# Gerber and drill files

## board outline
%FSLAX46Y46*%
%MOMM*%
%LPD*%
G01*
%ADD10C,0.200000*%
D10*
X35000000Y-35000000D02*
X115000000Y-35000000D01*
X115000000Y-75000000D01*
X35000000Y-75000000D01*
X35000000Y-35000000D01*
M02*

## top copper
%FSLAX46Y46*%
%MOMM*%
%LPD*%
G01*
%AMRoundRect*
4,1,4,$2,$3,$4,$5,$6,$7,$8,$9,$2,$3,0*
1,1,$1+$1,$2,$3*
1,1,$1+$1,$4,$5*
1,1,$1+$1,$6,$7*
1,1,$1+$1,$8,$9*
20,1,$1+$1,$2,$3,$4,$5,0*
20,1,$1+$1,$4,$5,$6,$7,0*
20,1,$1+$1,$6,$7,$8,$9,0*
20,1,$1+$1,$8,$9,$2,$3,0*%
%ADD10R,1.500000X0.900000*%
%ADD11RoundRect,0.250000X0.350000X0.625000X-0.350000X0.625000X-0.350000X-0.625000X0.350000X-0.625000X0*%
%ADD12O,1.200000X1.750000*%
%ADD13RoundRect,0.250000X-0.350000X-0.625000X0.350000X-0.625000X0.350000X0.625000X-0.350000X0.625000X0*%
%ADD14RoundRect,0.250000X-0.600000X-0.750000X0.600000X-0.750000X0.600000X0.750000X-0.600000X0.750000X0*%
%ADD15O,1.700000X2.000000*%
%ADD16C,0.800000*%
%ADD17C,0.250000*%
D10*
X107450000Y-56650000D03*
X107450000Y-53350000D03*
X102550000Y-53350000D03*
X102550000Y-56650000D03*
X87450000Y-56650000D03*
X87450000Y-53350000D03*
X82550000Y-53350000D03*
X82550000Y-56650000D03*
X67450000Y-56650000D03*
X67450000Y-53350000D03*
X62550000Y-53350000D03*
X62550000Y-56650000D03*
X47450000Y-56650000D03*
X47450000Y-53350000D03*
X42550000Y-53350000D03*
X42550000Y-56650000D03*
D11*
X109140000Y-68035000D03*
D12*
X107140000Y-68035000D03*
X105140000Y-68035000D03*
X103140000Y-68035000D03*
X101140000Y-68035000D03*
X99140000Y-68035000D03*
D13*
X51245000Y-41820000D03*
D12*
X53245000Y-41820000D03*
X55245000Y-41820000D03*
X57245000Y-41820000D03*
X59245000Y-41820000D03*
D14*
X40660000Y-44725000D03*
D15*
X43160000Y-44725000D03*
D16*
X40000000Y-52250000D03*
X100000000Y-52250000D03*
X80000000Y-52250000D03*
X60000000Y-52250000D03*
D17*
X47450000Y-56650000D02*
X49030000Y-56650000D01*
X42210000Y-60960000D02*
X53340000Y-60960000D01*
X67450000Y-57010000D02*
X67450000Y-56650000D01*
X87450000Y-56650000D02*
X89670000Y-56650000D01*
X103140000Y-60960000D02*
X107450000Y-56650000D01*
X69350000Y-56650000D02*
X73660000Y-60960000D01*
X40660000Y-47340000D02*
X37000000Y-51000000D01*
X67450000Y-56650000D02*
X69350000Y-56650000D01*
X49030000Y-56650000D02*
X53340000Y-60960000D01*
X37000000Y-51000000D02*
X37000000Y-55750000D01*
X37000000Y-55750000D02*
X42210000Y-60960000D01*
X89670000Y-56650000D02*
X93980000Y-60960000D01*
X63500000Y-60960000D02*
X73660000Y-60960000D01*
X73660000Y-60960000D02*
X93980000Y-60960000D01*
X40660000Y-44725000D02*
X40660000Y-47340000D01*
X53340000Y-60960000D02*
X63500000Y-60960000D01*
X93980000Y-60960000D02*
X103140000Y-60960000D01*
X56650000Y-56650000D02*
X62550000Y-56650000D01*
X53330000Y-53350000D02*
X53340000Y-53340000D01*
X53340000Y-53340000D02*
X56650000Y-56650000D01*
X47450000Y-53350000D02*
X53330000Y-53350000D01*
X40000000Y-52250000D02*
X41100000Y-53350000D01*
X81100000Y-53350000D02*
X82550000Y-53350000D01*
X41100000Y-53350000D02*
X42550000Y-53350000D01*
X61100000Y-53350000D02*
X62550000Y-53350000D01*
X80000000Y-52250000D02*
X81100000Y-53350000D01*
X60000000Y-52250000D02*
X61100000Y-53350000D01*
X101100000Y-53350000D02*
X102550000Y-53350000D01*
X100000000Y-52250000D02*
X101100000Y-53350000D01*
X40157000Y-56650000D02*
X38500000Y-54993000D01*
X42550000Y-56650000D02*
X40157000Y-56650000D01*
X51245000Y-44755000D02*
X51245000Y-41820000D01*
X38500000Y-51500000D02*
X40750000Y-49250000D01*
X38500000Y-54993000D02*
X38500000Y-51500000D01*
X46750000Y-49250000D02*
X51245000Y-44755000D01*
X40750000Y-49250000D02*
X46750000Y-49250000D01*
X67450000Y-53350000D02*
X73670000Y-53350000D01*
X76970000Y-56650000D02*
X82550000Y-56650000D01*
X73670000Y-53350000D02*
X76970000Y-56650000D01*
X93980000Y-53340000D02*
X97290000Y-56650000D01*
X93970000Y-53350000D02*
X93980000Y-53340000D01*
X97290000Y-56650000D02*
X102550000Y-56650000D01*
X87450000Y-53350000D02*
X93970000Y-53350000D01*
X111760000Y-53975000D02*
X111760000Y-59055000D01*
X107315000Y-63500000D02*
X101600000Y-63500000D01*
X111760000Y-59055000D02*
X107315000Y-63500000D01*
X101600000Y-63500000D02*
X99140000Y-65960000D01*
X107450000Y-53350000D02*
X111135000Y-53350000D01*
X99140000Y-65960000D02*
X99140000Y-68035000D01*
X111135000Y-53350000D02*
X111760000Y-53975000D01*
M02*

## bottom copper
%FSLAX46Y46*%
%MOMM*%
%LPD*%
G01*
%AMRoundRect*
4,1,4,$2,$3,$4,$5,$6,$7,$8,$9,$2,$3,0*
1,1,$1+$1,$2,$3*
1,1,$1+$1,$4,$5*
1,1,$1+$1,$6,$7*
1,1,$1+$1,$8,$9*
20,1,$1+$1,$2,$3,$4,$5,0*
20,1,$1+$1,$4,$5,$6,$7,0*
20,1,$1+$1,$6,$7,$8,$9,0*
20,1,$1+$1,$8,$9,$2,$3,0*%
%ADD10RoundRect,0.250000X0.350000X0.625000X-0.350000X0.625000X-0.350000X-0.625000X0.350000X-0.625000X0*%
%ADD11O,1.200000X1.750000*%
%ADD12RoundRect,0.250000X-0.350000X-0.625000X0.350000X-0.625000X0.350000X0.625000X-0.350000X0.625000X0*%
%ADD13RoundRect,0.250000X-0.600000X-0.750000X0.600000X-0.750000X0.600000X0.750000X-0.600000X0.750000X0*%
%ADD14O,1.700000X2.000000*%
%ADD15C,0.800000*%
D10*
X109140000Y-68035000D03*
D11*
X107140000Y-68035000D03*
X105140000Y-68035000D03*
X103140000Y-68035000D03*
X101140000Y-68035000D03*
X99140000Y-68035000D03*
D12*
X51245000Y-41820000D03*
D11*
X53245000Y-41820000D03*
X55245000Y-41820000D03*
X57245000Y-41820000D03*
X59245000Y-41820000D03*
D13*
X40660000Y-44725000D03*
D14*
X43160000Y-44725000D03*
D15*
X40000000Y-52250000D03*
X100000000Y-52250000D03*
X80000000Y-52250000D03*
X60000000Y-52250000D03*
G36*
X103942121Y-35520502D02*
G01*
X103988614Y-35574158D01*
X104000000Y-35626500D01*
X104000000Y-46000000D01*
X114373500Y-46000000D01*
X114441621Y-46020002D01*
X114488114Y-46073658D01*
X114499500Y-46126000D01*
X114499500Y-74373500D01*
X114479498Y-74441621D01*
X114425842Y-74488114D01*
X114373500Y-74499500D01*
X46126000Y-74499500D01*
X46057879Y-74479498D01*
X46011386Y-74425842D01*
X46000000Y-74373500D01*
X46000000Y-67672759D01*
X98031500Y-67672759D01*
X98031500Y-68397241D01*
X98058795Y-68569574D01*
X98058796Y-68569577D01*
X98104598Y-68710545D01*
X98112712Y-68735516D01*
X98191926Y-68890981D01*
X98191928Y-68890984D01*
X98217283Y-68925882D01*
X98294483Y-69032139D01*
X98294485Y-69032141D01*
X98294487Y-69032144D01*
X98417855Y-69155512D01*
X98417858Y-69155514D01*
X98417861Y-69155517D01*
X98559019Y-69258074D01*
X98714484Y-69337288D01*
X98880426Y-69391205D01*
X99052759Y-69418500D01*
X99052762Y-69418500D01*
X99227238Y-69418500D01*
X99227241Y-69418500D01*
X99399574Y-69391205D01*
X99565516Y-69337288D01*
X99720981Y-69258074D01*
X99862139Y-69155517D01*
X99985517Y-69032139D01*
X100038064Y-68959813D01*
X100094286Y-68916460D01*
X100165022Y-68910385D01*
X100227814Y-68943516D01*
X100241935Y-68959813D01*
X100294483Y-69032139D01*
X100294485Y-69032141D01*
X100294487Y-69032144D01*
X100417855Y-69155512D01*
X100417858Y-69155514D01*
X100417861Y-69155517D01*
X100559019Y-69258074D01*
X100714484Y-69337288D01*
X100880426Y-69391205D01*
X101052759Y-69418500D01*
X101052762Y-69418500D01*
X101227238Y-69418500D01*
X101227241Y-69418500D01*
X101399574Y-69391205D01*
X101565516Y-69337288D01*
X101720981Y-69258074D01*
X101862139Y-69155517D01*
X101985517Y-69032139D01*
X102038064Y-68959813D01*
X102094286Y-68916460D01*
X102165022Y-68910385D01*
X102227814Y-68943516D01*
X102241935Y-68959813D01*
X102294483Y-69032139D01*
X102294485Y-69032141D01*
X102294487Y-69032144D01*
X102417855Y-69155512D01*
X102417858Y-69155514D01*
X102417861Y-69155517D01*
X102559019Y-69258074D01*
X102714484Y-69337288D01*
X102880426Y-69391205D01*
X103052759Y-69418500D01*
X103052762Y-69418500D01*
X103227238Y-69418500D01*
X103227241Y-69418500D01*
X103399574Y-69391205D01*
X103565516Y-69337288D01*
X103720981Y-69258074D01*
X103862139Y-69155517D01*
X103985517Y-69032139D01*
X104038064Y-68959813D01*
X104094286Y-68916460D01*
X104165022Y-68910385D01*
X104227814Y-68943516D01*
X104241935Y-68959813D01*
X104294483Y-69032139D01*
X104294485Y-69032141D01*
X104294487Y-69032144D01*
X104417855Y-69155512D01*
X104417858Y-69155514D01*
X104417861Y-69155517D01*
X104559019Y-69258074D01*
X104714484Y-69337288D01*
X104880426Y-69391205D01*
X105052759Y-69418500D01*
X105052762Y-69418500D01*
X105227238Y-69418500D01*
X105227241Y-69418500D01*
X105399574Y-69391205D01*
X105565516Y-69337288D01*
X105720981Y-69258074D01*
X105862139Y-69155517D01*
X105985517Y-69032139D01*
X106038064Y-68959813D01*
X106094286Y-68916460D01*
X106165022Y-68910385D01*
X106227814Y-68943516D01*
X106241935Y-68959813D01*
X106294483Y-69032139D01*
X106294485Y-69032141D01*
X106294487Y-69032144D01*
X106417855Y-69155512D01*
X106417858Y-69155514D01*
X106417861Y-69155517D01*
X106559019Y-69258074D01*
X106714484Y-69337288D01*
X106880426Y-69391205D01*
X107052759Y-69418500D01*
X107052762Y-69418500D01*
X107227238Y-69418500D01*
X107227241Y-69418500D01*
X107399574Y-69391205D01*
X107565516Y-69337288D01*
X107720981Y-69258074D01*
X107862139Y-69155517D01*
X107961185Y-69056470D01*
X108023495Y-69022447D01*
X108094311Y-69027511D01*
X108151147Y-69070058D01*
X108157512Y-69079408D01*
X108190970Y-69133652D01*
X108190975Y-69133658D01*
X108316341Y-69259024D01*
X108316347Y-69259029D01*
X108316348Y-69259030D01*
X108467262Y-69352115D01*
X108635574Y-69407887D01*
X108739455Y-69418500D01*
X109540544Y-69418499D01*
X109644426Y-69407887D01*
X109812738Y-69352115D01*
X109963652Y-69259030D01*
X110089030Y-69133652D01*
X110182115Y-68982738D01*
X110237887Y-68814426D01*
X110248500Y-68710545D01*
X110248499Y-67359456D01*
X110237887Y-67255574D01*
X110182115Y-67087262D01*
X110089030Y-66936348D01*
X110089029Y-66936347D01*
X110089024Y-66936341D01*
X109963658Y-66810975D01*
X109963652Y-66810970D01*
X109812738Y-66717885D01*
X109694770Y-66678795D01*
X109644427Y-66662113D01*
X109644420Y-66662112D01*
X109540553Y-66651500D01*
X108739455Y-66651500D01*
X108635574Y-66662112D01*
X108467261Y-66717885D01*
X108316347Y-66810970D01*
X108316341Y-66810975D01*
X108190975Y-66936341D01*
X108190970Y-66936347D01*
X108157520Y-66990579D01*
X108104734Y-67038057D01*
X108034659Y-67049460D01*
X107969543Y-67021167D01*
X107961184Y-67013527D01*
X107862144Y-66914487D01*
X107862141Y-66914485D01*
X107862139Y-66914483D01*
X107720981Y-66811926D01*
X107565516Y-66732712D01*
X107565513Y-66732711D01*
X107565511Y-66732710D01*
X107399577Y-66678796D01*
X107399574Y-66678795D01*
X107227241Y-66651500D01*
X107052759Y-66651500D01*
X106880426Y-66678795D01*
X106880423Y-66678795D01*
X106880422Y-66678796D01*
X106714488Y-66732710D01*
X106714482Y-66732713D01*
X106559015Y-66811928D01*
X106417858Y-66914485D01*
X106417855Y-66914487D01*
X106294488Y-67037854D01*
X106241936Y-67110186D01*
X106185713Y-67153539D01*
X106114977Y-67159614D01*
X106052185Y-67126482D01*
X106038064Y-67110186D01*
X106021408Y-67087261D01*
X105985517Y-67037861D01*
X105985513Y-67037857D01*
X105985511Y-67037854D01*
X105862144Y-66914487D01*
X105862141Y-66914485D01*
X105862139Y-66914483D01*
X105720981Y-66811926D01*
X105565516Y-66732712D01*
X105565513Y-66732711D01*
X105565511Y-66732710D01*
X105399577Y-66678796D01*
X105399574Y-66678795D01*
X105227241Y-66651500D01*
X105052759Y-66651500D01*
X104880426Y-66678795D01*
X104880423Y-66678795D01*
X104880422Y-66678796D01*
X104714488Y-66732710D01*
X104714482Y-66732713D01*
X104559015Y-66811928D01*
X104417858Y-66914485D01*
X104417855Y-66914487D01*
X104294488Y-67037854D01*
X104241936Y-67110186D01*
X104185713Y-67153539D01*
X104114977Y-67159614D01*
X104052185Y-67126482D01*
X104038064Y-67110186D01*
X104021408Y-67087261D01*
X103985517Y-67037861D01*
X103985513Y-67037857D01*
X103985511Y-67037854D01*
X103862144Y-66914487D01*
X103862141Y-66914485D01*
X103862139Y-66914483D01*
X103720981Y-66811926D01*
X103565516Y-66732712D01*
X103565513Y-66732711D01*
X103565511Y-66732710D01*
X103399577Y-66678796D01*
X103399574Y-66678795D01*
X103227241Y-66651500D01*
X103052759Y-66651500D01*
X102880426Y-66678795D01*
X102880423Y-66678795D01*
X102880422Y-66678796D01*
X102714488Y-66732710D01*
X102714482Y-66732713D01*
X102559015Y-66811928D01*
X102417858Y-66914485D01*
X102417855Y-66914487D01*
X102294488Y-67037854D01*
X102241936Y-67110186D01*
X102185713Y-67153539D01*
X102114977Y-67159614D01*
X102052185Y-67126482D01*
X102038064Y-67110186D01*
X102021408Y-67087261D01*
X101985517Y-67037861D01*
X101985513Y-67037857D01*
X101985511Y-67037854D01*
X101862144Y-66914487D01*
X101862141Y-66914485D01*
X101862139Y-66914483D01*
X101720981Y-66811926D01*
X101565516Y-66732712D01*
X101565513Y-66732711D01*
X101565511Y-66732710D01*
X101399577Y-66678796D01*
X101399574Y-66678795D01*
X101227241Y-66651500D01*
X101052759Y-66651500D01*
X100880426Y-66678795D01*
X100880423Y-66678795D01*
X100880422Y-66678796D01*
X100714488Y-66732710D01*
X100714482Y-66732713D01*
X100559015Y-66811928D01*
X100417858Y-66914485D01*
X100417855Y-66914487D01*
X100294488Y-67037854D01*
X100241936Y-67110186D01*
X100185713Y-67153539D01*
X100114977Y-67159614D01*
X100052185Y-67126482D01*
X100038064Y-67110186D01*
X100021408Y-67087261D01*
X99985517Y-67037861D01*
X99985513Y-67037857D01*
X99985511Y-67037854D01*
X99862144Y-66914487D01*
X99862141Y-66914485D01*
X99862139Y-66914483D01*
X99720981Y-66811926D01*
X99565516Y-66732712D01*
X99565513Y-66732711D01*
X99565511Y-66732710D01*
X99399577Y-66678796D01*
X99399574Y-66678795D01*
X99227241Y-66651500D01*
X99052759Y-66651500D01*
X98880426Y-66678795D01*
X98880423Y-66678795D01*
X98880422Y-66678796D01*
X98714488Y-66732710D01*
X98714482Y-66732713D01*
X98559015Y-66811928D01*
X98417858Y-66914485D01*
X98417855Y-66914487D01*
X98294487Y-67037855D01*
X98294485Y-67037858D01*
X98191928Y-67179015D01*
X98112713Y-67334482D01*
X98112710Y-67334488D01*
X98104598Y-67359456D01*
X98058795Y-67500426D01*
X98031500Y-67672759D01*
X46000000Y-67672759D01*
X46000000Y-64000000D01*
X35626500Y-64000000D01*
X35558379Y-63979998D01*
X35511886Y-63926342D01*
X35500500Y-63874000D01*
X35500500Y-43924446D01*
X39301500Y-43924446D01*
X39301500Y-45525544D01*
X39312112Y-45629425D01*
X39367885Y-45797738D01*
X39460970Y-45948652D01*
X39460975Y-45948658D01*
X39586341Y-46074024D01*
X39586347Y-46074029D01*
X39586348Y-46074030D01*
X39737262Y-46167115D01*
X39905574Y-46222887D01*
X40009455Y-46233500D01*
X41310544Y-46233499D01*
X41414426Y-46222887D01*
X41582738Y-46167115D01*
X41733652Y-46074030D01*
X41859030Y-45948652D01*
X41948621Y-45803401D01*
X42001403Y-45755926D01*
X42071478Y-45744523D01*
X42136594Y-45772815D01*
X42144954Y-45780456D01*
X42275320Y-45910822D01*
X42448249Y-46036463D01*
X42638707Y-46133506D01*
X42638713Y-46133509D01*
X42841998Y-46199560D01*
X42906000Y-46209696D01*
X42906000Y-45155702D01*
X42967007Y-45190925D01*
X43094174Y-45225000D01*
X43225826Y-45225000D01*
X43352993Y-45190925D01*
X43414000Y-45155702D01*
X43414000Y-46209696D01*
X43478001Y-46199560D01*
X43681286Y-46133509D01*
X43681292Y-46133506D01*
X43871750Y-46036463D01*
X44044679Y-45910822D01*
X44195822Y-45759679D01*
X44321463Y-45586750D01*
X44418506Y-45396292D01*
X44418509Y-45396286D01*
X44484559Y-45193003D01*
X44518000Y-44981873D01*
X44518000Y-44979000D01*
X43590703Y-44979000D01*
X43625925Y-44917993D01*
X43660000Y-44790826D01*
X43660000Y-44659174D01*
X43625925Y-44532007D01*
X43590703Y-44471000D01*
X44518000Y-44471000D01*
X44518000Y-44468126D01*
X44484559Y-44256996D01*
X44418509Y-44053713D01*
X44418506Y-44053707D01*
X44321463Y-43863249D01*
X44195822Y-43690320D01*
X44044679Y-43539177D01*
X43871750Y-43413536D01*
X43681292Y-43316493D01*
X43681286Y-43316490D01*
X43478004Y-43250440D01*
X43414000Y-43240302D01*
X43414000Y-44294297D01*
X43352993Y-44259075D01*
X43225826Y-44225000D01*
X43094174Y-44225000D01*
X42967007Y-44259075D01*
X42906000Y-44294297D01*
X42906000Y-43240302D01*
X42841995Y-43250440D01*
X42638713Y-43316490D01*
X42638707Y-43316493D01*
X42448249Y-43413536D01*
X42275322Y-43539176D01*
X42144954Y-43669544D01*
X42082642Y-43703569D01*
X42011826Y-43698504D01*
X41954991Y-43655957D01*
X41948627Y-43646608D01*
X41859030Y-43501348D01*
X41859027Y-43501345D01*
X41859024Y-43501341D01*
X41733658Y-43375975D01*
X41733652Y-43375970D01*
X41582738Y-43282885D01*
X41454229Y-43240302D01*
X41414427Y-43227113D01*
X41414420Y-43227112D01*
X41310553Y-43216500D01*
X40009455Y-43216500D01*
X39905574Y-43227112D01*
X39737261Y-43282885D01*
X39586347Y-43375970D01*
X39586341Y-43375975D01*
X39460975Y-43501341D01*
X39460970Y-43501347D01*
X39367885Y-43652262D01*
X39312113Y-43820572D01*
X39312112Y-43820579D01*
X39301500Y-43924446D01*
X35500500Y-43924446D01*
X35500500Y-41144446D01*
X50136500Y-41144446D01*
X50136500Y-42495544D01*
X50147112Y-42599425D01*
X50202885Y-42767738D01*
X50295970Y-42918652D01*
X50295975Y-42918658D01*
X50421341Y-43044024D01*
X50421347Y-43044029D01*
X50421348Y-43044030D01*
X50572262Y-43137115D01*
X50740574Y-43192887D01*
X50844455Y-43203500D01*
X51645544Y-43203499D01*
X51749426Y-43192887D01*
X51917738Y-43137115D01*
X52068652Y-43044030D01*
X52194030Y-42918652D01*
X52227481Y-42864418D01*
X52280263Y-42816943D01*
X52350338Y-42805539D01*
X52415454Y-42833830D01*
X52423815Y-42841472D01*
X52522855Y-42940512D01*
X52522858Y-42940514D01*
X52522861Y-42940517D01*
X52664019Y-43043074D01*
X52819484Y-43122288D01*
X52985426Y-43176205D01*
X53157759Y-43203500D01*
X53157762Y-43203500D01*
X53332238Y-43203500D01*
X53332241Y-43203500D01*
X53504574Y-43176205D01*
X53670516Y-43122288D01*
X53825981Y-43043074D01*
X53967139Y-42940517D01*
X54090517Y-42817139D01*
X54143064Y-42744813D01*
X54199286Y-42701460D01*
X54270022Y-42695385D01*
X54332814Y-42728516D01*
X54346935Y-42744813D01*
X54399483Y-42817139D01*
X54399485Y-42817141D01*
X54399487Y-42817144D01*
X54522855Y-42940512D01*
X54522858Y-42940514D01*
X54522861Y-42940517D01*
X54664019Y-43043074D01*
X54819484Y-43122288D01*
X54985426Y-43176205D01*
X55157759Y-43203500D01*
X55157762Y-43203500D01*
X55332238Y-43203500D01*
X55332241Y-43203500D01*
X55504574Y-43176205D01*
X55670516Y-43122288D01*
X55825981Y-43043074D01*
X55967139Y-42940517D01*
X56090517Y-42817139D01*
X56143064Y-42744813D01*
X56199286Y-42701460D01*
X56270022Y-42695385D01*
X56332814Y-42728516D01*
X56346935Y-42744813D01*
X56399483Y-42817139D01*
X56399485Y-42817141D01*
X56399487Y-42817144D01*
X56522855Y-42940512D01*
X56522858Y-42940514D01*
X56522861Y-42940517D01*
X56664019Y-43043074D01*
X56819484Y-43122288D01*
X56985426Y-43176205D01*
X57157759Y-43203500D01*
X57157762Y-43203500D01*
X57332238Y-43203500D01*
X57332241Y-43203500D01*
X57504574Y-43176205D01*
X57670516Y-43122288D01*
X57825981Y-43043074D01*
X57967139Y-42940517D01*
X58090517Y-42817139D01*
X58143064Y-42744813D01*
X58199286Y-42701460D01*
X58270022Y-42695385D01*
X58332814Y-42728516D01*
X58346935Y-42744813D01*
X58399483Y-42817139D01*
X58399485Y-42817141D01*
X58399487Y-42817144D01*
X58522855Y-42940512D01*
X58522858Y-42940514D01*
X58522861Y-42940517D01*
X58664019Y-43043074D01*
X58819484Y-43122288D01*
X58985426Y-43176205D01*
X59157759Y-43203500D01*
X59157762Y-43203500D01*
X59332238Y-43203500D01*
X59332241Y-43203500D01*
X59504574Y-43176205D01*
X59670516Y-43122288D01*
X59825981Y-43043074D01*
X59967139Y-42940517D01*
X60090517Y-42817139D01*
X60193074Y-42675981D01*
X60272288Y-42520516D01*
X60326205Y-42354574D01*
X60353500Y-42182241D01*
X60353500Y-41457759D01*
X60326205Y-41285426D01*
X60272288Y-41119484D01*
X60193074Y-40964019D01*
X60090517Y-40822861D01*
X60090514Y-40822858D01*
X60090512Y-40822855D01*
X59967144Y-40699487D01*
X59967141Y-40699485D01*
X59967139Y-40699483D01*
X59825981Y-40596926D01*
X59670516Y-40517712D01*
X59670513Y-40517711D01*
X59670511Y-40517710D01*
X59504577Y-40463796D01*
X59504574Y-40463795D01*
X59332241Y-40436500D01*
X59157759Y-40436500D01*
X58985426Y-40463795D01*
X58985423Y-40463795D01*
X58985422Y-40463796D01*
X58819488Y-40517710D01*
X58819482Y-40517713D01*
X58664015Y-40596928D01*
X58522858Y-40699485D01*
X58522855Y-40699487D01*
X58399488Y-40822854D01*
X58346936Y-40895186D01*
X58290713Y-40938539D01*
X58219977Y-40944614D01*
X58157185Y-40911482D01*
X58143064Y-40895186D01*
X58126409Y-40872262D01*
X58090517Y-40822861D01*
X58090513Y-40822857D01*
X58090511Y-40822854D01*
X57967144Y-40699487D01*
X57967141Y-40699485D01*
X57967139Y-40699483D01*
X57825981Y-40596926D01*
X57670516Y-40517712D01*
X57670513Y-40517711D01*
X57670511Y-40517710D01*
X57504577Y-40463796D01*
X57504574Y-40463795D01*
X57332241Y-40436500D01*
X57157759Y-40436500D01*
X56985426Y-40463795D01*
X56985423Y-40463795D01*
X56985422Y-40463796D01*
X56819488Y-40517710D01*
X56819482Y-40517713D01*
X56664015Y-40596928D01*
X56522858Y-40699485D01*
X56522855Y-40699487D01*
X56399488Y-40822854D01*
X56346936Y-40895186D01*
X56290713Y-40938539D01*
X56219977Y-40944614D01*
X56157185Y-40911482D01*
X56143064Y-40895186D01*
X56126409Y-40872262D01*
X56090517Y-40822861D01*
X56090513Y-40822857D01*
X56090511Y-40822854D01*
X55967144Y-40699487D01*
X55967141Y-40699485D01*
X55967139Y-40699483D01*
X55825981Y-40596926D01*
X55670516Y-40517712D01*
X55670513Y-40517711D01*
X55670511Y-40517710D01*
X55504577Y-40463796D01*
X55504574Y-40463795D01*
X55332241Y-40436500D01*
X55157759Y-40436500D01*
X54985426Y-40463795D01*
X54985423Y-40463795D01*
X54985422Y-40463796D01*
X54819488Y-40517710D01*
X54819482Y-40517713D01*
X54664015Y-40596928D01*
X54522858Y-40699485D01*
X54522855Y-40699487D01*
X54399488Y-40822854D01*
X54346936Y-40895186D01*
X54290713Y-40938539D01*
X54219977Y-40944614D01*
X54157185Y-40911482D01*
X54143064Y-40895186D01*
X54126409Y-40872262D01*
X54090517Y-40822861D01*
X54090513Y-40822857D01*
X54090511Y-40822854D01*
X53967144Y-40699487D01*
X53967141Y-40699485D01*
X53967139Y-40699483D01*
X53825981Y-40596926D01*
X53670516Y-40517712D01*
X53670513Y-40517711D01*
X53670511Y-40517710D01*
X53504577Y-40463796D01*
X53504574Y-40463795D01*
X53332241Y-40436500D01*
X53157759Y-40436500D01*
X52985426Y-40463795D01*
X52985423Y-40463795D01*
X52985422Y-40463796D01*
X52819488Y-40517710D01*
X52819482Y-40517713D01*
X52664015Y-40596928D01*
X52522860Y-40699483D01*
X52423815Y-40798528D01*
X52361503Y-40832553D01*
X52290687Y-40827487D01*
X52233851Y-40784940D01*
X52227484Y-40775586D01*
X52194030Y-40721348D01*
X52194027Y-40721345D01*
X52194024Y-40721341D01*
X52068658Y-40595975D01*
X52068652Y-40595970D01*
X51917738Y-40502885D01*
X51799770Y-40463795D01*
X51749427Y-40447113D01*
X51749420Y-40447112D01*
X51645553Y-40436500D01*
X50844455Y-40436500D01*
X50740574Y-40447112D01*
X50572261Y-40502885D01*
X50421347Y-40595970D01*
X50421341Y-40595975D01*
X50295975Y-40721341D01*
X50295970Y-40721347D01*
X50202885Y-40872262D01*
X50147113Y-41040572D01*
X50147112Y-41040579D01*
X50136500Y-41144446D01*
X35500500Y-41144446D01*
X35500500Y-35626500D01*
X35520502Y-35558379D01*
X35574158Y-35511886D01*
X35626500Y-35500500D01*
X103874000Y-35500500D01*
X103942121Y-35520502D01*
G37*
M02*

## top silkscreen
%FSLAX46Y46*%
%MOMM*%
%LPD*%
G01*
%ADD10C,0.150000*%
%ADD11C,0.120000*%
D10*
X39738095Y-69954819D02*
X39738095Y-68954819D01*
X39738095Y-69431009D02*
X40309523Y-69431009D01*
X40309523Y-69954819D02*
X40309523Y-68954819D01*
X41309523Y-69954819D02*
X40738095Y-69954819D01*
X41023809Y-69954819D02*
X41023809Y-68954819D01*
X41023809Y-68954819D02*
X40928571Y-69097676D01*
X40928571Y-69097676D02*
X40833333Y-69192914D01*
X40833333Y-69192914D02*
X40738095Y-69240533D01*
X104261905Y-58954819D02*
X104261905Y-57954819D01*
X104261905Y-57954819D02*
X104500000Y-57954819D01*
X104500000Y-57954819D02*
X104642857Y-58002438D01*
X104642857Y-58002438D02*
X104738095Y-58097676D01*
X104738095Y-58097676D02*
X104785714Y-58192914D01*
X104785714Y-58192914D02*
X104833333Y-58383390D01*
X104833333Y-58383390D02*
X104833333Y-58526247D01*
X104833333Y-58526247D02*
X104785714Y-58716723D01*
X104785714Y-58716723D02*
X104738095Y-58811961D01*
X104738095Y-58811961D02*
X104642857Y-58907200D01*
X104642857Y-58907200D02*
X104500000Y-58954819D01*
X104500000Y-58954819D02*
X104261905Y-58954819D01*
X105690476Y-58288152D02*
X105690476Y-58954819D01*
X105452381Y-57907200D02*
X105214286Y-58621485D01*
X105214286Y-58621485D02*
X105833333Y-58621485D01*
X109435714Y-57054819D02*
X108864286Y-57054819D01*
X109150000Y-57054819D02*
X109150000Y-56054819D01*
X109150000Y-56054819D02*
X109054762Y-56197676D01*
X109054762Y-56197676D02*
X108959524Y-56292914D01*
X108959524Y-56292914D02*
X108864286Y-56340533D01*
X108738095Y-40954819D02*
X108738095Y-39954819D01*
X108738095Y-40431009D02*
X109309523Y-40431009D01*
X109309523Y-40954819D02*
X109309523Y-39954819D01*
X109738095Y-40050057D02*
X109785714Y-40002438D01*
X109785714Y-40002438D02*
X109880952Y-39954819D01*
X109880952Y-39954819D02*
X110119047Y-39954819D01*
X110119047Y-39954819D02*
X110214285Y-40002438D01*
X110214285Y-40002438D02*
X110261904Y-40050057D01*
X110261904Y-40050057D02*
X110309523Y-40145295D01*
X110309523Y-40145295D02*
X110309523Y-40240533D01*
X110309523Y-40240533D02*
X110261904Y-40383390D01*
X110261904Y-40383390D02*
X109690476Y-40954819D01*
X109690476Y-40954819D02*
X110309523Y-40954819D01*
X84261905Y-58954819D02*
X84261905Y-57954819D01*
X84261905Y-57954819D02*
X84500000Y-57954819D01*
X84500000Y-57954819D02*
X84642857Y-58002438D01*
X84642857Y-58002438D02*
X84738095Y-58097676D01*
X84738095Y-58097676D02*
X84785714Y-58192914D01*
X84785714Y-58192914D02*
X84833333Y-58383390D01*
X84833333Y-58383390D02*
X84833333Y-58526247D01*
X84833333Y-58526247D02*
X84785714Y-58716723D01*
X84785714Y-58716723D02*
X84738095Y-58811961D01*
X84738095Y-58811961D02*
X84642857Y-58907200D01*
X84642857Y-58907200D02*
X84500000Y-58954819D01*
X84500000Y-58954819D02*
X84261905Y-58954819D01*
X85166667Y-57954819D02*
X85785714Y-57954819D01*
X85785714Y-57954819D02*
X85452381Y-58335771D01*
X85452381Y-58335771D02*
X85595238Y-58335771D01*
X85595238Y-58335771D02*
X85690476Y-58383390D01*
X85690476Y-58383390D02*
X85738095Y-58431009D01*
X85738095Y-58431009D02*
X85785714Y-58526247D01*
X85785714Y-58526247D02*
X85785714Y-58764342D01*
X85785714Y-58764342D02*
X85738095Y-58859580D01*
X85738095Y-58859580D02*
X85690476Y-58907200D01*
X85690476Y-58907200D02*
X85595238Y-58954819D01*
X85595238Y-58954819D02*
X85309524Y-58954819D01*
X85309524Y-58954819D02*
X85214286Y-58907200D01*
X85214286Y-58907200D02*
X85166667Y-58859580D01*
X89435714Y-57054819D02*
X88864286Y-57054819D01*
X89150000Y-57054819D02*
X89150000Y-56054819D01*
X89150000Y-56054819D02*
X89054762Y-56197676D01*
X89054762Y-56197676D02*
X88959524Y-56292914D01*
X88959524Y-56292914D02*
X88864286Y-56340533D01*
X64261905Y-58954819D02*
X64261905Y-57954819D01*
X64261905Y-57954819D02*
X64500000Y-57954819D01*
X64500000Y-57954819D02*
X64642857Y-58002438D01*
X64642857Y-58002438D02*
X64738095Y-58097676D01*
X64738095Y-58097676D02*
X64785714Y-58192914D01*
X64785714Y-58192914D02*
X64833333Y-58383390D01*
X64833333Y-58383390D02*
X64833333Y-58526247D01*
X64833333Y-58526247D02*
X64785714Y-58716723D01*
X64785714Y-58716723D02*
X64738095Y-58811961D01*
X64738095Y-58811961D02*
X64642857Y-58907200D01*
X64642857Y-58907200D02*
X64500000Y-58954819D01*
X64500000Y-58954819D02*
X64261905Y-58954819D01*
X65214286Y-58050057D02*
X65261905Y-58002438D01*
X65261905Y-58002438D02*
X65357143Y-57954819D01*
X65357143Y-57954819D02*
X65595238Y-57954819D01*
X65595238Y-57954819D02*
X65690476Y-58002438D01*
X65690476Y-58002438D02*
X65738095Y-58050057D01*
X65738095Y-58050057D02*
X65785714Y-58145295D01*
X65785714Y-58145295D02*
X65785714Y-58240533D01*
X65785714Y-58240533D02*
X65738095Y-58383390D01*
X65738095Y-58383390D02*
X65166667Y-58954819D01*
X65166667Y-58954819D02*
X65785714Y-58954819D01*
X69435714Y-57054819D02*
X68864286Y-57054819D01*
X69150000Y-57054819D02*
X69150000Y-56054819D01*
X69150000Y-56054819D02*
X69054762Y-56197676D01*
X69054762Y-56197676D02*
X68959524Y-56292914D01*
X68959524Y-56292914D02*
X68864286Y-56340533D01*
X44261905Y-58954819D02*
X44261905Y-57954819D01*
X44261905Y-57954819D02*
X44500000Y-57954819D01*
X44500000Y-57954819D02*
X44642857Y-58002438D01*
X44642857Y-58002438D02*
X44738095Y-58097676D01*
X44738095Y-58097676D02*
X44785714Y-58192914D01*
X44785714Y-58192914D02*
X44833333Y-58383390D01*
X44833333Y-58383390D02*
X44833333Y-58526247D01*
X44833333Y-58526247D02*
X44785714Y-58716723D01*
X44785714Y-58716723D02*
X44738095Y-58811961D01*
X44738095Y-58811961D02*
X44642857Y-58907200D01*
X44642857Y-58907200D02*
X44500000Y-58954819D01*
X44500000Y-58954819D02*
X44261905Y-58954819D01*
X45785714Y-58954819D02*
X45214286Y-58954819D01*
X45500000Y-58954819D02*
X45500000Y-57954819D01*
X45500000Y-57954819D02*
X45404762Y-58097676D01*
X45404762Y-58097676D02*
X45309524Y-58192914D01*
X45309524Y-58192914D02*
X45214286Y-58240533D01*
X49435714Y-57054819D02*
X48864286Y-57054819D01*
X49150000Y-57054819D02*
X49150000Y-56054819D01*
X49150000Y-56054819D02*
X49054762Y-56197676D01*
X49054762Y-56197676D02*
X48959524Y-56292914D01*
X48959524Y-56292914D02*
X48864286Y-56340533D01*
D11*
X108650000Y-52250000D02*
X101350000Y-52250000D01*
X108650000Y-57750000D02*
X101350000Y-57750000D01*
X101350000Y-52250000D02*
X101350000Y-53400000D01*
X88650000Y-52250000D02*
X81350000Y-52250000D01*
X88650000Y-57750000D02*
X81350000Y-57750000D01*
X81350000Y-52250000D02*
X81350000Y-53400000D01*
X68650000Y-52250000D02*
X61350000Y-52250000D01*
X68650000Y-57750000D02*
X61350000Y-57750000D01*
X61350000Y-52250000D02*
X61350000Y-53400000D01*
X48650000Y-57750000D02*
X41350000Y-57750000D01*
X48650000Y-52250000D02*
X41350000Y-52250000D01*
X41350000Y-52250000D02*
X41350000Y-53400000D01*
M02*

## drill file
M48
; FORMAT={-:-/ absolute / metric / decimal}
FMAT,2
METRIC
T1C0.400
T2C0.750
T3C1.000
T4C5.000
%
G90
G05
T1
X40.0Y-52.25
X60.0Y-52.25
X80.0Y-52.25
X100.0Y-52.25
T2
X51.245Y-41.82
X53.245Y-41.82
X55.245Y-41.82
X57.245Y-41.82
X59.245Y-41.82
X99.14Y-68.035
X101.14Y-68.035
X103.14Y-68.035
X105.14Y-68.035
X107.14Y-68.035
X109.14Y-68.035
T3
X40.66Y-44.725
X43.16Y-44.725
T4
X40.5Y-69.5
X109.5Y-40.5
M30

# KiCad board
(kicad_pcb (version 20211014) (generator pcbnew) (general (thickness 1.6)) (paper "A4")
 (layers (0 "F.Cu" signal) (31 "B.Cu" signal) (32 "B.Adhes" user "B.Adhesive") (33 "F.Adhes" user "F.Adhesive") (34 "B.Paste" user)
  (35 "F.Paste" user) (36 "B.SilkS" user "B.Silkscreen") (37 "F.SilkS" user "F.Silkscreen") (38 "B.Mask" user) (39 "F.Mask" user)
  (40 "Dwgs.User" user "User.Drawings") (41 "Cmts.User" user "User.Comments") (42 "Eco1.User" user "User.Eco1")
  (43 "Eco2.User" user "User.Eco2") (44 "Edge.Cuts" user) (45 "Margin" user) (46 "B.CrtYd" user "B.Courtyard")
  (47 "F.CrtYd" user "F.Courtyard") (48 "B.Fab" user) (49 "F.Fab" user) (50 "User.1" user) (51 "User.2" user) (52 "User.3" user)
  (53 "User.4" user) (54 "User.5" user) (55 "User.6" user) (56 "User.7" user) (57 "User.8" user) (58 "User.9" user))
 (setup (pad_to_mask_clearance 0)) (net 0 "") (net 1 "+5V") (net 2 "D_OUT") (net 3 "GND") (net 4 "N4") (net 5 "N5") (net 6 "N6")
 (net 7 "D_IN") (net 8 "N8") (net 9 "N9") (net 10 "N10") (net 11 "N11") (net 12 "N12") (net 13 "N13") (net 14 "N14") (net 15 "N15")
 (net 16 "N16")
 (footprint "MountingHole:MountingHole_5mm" (layer "F.Cu") (at 40.5 69.5)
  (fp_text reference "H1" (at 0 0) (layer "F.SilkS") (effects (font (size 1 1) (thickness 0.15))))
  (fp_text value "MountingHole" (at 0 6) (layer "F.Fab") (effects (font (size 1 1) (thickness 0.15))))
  (pad "" np_thru_hole circle (at 0 0) (size 5 5) (drill 5) (layers *.Cu *.Mask)))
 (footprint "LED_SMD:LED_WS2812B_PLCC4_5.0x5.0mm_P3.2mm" (layer "F.Cu") (at 105 55 180)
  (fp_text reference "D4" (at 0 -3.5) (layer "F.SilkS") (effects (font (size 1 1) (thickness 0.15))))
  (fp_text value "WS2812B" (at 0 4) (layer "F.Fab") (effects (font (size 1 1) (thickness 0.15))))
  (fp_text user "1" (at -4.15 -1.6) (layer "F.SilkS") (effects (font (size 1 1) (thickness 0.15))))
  (fp_line (start -3.65 2.75) (end 3.65 2.75) (layer "F.SilkS") (width 0.12))
  (fp_line (start -3.65 -2.75) (end 3.65 -2.75) (layer "F.SilkS") (width 0.12))
  (fp_line (start 3.65 2.75) (end 3.65 1.6) (layer "F.SilkS") (width 0.12))
  (pad "1" smd rect (at -2.45 -1.65 180) (size 1.5 0.9) (layers "F.Cu" "F.Paste" "F.Mask") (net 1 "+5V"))
  (pad "2" smd rect (at -2.45 1.65 180) (size 1.5 0.9) (layers "F.Cu" "F.Paste" "F.Mask") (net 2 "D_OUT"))
  (pad "3" smd rect (at 2.45 1.65 180) (size 1.5 0.9) (layers "F.Cu" "F.Paste" "F.Mask") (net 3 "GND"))
  (pad "4" smd rect (at 2.45 -1.65 180) (size 1.5 0.9) (layers "F.Cu" "F.Paste" "F.Mask") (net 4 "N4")))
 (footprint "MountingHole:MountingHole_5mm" (layer "F.Cu") (at 109.5 40.5)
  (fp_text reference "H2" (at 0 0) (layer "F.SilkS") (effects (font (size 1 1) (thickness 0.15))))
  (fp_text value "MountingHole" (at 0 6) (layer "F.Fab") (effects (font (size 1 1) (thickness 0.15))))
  (pad "" np_thru_hole circle (at 0 0) (size 5 5) (drill 5) (layers *.Cu *.Mask)))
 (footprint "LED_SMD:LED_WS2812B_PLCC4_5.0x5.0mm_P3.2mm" (layer "F.Cu") (at 85 55 180)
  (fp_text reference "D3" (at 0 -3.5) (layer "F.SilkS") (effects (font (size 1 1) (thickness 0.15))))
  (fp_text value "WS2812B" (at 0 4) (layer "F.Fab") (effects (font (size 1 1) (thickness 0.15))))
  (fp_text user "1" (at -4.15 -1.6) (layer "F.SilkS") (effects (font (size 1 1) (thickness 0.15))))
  (fp_line (start -3.65 2.75) (end 3.65 2.75) (layer "F.SilkS") (width 0.12))
  (fp_line (start -3.65 -2.75) (end 3.65 -2.75) (layer "F.SilkS") (width 0.12))
  (fp_line (start 3.65 2.75) (end 3.65 1.6) (layer "F.SilkS") (width 0.12))
  (pad "1" smd rect (at -2.45 -1.65 180) (size 1.5 0.9) (layers "F.Cu" "F.Paste" "F.Mask") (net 1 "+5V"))
  (pad "2" smd rect (at -2.45 1.65 180) (size 1.5 0.9) (layers "F.Cu" "F.Paste" "F.Mask") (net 4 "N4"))
  (pad "3" smd rect (at 2.45 1.65 180) (size 1.5 0.9) (layers "F.Cu" "F.Paste" "F.Mask") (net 3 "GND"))
  (pad "4" smd rect (at 2.45 -1.65 180) (size 1.5 0.9) (layers "F.Cu" "F.Paste" "F.Mask") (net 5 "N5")))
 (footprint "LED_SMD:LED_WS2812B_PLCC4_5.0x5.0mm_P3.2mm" (layer "F.Cu") (at 65 55 180)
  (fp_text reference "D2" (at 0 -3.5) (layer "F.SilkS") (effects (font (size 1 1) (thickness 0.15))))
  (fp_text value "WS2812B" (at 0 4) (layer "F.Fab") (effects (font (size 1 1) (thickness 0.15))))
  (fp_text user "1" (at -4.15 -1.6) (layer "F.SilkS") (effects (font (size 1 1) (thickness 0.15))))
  (fp_line (start -3.65 2.75) (end 3.65 2.75) (layer "F.SilkS") (width 0.12))
  (fp_line (start -3.65 -2.75) (end 3.65 -2.75) (layer "F.SilkS") (width 0.12))
  (fp_line (start 3.65 2.75) (end 3.65 1.6) (layer "F.SilkS") (width 0.12))
  (pad "1" smd rect (at -2.45 -1.65 180) (size 1.5 0.9) (layers "F.Cu" "F.Paste" "F.Mask") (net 1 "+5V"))
  (pad "2" smd rect (at -2.45 1.65 180) (size 1.5 0.9) (layers "F.Cu" "F.Paste" "F.Mask") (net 5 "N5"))
  (pad "3" smd rect (at 2.45 1.65 180) (size 1.5 0.9) (layers "F.Cu" "F.Paste" "F.Mask") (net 3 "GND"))
  (pad "4" smd rect (at 2.45 -1.65 180) (size 1.5 0.9) (layers "F.Cu" "F.Paste" "F.Mask") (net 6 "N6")))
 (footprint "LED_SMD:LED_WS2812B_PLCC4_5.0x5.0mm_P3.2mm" (layer "F.Cu") (at 45 55 180)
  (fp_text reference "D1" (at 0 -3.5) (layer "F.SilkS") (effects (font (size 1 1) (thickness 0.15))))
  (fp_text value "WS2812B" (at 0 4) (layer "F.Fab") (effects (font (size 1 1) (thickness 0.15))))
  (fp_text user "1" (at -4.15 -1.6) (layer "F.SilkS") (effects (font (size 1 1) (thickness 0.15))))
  (fp_line (start -3.65 -2.75) (end 3.65 -2.75) (layer "F.SilkS") (width 0.12))
  (fp_line (start -3.65 2.75) (end 3.65 2.75) (layer "F.SilkS") (width 0.12))
  (fp_line (start 3.65 2.75) (end 3.65 1.6) (layer "F.SilkS") (width 0.12))
  (pad "1" smd rect (at -2.45 -1.65 180) (size 1.5 0.9) (layers "F.Cu" "F.Paste" "F.Mask") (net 1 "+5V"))
  (pad "2" smd rect (at -2.45 1.65 180) (size 1.5 0.9) (layers "F.Cu" "F.Paste" "F.Mask") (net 6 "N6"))
  (pad "3" smd rect (at 2.45 1.65 180) (size 1.5 0.9) (layers "F.Cu" "F.Paste" "F.Mask") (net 3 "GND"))
  (pad "4" smd rect (at 2.45 -1.65 180) (size 1.5 0.9) (layers "F.Cu" "F.Paste" "F.Mask") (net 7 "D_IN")))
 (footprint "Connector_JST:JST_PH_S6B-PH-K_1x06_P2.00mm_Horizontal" (layer "B.Cu") (at 109.14 68.035 180)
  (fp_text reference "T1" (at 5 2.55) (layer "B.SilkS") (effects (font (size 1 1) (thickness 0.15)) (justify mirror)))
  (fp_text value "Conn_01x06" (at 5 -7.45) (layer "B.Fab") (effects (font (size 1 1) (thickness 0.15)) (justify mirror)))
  (pad "1" thru_hole roundrect (at 0 0 180) (size 1.2 1.75) (drill 0.75) (layers *.Cu *.Mask) (roundrect_rratio 0.2083333333) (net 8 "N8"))
  (pad "2" thru_hole oval (at 2 0 180) (size 1.2 1.75) (drill 0.75) (layers *.Cu *.Mask) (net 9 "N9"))
  (pad "3" thru_hole oval (at 4 0 180) (size 1.2 1.75) (drill 0.75) (layers *.Cu *.Mask) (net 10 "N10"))
  (pad "4" thru_hole oval (at 6 0 180) (size 1.2 1.75) (drill 0.75) (layers *.Cu *.Mask) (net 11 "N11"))
  (pad "5" thru_hole oval (at 8 0 180) (size 1.2 1.75) (drill 0.75) (layers *.Cu *.Mask) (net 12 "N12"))
  (pad "6" thru_hole oval (at 10 0 180) (size 1.2 1.75) (drill 0.75) (layers *.Cu *.Mask) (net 2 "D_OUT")))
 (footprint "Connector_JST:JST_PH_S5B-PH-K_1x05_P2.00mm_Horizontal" (layer "B.Cu") (at 51.245 41.82)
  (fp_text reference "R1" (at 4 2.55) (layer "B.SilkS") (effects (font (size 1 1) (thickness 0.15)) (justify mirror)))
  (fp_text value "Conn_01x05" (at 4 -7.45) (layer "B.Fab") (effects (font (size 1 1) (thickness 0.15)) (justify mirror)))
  (pad "1" thru_hole roundrect (at 0 0) (size 1.2 1.75) (drill 0.75) (layers *.Cu *.Mask) (roundrect_rratio 0.2083333333) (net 7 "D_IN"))
  (pad "2" thru_hole oval (at 2 0) (size 1.2 1.75) (drill 0.75) (layers *.Cu *.Mask) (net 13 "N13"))
  (pad "3" thru_hole oval (at 4 0) (size 1.2 1.75) (drill 0.75) (layers *.Cu *.Mask) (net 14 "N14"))
  (pad "4" thru_hole oval (at 6 0) (size 1.2 1.75) (drill 0.75) (layers *.Cu *.Mask) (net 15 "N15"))
  (pad "5" thru_hole oval (at 8 0) (size 1.2 1.75) (drill 0.75) (layers *.Cu *.Mask) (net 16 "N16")))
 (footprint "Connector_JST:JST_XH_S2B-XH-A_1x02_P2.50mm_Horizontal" (layer "B.Cu") (at 40.66 44.725)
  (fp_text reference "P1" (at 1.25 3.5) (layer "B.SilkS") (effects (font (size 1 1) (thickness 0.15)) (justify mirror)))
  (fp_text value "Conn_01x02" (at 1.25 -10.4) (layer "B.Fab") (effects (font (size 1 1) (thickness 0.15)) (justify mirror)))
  (pad "1" thru_hole roundrect (at 0 0) (size 1.7 2) (drill 1) (layers *.Cu *.Mask) (roundrect_rratio 0.1470588235) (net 1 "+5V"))
  (pad "2" thru_hole oval (at 2.5 0) (size 1.7 2) (drill 1) (layers *.Cu *.Mask) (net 3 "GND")))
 (gr_rect (start 35 35) (end 115 75) (layer "Edge.Cuts") (width 0.2) (fill none))
 (segment (start 47.45 56.65) (end 49.03 56.65) (width 0.25) (layer "F.Cu") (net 1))
 (segment (start 42.21 60.96) (end 53.34 60.96) (width 0.25) (layer "F.Cu") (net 1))
 (segment (start 67.45 57.01) (end 67.45 56.65) (width 0.25) (layer "F.Cu") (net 1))
 (segment (start 87.45 56.65) (end 89.67 56.65) (width 0.25) (layer "F.Cu") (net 1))
 (segment (start 103.14 60.96) (end 107.45 56.65) (width 0.25) (layer "F.Cu") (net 1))
 (segment (start 69.35 56.65) (end 73.66 60.96) (width 0.25) (layer "F.Cu") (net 1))
 (segment (start 40.66 47.34) (end 37 51) (width 0.25) (layer "F.Cu") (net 1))
 (segment (start 67.45 56.65) (end 69.35 56.65) (width 0.25) (layer "F.Cu") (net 1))
 (segment (start 49.03 56.65) (end 53.34 60.96) (width 0.25) (layer "F.Cu") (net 1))
 (segment (start 37 51) (end 37 55.75) (width 0.25) (layer "F.Cu") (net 1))
 (segment (start 37 55.75) (end 42.21 60.96) (width 0.25) (layer "F.Cu") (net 1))
 (segment (start 89.67 56.65) (end 93.98 60.96) (width 0.25) (layer "F.Cu") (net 1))
 (segment (start 63.5 60.96) (end 73.66 60.96) (width 0.25) (layer "F.Cu") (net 1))
 (segment (start 73.66 60.96) (end 93.98 60.96) (width 0.25) (layer "F.Cu") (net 1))
 (segment (start 40.66 44.725) (end 40.66 47.34) (width 0.25) (layer "F.Cu") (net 1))
 (segment (start 53.34 60.96) (end 63.5 60.96) (width 0.25) (layer "F.Cu") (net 1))
 (segment (start 93.98 60.96) (end 103.14 60.96) (width 0.25) (layer "F.Cu") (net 1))
 (segment (start 56.65 56.65) (end 62.55 56.65) (width 0.25) (layer "F.Cu") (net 6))
 (segment (start 53.33 53.35) (end 53.34 53.34) (width 0.25) (layer "F.Cu") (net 6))
 (segment (start 53.34 53.34) (end 56.65 56.65) (width 0.25) (layer "F.Cu") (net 6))
 (segment (start 47.45 53.35) (end 53.33 53.35) (width 0.25) (layer "F.Cu") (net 6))
 (segment (start 40 52.25) (end 41.1 53.35) (width 0.25) (layer "F.Cu") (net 3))
 (segment (start 81.1 53.35) (end 82.55 53.35) (width 0.25) (layer "F.Cu") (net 3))
 (segment (start 41.1 53.35) (end 42.55 53.35) (width 0.25) (layer "F.Cu") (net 3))
 (segment (start 61.1 53.35) (end 62.55 53.35) (width 0.25) (layer "F.Cu") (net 3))
 (segment (start 80 52.25) (end 81.1 53.35) (width 0.25) (layer "F.Cu") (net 3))
 (segment (start 60 52.25) (end 61.1 53.35) (width 0.25) (layer "F.Cu") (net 3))
 (segment (start 101.1 53.35) (end 102.55 53.35) (width 0.25) (layer "F.Cu") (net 3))
 (segment (start 100 52.25) (end 101.1 53.35) (width 0.25) (layer "F.Cu") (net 3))
 (via (at 40 52.25) (size 0.8) (drill 0.4) (layers "F.Cu" "B.Cu") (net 3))
 (via (at 100 52.25) (size 0.8) (drill 0.4) (layers "F.Cu" "B.Cu") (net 3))
 (via (at 80 52.25) (size 0.8) (drill 0.4) (layers "F.Cu" "B.Cu") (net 3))
 (via (at 60 52.25) (size 0.8) (drill 0.4) (layers "F.Cu" "B.Cu") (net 3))
 (segment (start 40.157 56.65) (end 38.5 54.993) (width 0.25) (layer "F.Cu") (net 7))
 (segment (start 42.55 56.65) (end 40.157 56.65) (width 0.25) (layer "F.Cu") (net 7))
 (segment (start 51.245 44.755) (end 51.245 41.82) (width 0.25) (layer "F.Cu") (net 7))
 (segment (start 38.5 51.5) (end 40.75 49.25) (width 0.25) (layer "F.Cu") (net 7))
 (segment (start 38.5 54.993) (end 38.5 51.5) (width 0.25) (layer "F.Cu") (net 7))
 (segment (start 46.75 49.25) (end 51.245 44.755) (width 0.25) (layer "F.Cu") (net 7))
 (segment (start 40.75 49.25) (end 46.75 49.25) (width 0.25) (layer "F.Cu") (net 7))
 (segment (start 67.45 53.35) (end 73.67 53.35) (width 0.25) (layer "F.Cu") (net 5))
 (segment (start 76.97 56.65) (end 82.55 56.65) (width 0.25) (layer "F.Cu") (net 5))
 (segment (start 73.67 53.35) (end 76.97 56.65) (width 0.25) (layer "F.Cu") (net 5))
 (segment (start 93.98 53.34) (end 97.29 56.65) (width 0.25) (layer "F.Cu") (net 4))
 (segment (start 93.97 53.35) (end 93.98 53.34) (width 0.25) (layer "F.Cu") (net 4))
 (segment (start 97.29 56.65) (end 102.55 56.65) (width 0.25) (layer "F.Cu") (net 4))
 (segment (start 87.45 53.35) (end 93.97 53.35) (width 0.25) (layer "F.Cu") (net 4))
 (segment (start 111.76 53.975) (end 111.76 59.055) (width 0.25) (layer "F.Cu") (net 2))
 (segment (start 107.315 63.5) (end 101.6 63.5) (width 0.25) (layer "F.Cu") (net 2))
 (segment (start 111.76 59.055) (end 107.315 63.5) (width 0.25) (layer "F.Cu") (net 2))
 (segment (start 101.6 63.5) (end 99.14 65.96) (width 0.25) (layer "F.Cu") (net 2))
 (segment (start 107.45 53.35) (end 111.135 53.35) (width 0.25) (layer "F.Cu") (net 2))
 (segment (start 99.14 65.96) (end 99.14 68.035) (width 0.25) (layer "F.Cu") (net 2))
 (segment (start 111.135 53.35) (end 111.76 53.975) (width 0.25) (layer "F.Cu") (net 2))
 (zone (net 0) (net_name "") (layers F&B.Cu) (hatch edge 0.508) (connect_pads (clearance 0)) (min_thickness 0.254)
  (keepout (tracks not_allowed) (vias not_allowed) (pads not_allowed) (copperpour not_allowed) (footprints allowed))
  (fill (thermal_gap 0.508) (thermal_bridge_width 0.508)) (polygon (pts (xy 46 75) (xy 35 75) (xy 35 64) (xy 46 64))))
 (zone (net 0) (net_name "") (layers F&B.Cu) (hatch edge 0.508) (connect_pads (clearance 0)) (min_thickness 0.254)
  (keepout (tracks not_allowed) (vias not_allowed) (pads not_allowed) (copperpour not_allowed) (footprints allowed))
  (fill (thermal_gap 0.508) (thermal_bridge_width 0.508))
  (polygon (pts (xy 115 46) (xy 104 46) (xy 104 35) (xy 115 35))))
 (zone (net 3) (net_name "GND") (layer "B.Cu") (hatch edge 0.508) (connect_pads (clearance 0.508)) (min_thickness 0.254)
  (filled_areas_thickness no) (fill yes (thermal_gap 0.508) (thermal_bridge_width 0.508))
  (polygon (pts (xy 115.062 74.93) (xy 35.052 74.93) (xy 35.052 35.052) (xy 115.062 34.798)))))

